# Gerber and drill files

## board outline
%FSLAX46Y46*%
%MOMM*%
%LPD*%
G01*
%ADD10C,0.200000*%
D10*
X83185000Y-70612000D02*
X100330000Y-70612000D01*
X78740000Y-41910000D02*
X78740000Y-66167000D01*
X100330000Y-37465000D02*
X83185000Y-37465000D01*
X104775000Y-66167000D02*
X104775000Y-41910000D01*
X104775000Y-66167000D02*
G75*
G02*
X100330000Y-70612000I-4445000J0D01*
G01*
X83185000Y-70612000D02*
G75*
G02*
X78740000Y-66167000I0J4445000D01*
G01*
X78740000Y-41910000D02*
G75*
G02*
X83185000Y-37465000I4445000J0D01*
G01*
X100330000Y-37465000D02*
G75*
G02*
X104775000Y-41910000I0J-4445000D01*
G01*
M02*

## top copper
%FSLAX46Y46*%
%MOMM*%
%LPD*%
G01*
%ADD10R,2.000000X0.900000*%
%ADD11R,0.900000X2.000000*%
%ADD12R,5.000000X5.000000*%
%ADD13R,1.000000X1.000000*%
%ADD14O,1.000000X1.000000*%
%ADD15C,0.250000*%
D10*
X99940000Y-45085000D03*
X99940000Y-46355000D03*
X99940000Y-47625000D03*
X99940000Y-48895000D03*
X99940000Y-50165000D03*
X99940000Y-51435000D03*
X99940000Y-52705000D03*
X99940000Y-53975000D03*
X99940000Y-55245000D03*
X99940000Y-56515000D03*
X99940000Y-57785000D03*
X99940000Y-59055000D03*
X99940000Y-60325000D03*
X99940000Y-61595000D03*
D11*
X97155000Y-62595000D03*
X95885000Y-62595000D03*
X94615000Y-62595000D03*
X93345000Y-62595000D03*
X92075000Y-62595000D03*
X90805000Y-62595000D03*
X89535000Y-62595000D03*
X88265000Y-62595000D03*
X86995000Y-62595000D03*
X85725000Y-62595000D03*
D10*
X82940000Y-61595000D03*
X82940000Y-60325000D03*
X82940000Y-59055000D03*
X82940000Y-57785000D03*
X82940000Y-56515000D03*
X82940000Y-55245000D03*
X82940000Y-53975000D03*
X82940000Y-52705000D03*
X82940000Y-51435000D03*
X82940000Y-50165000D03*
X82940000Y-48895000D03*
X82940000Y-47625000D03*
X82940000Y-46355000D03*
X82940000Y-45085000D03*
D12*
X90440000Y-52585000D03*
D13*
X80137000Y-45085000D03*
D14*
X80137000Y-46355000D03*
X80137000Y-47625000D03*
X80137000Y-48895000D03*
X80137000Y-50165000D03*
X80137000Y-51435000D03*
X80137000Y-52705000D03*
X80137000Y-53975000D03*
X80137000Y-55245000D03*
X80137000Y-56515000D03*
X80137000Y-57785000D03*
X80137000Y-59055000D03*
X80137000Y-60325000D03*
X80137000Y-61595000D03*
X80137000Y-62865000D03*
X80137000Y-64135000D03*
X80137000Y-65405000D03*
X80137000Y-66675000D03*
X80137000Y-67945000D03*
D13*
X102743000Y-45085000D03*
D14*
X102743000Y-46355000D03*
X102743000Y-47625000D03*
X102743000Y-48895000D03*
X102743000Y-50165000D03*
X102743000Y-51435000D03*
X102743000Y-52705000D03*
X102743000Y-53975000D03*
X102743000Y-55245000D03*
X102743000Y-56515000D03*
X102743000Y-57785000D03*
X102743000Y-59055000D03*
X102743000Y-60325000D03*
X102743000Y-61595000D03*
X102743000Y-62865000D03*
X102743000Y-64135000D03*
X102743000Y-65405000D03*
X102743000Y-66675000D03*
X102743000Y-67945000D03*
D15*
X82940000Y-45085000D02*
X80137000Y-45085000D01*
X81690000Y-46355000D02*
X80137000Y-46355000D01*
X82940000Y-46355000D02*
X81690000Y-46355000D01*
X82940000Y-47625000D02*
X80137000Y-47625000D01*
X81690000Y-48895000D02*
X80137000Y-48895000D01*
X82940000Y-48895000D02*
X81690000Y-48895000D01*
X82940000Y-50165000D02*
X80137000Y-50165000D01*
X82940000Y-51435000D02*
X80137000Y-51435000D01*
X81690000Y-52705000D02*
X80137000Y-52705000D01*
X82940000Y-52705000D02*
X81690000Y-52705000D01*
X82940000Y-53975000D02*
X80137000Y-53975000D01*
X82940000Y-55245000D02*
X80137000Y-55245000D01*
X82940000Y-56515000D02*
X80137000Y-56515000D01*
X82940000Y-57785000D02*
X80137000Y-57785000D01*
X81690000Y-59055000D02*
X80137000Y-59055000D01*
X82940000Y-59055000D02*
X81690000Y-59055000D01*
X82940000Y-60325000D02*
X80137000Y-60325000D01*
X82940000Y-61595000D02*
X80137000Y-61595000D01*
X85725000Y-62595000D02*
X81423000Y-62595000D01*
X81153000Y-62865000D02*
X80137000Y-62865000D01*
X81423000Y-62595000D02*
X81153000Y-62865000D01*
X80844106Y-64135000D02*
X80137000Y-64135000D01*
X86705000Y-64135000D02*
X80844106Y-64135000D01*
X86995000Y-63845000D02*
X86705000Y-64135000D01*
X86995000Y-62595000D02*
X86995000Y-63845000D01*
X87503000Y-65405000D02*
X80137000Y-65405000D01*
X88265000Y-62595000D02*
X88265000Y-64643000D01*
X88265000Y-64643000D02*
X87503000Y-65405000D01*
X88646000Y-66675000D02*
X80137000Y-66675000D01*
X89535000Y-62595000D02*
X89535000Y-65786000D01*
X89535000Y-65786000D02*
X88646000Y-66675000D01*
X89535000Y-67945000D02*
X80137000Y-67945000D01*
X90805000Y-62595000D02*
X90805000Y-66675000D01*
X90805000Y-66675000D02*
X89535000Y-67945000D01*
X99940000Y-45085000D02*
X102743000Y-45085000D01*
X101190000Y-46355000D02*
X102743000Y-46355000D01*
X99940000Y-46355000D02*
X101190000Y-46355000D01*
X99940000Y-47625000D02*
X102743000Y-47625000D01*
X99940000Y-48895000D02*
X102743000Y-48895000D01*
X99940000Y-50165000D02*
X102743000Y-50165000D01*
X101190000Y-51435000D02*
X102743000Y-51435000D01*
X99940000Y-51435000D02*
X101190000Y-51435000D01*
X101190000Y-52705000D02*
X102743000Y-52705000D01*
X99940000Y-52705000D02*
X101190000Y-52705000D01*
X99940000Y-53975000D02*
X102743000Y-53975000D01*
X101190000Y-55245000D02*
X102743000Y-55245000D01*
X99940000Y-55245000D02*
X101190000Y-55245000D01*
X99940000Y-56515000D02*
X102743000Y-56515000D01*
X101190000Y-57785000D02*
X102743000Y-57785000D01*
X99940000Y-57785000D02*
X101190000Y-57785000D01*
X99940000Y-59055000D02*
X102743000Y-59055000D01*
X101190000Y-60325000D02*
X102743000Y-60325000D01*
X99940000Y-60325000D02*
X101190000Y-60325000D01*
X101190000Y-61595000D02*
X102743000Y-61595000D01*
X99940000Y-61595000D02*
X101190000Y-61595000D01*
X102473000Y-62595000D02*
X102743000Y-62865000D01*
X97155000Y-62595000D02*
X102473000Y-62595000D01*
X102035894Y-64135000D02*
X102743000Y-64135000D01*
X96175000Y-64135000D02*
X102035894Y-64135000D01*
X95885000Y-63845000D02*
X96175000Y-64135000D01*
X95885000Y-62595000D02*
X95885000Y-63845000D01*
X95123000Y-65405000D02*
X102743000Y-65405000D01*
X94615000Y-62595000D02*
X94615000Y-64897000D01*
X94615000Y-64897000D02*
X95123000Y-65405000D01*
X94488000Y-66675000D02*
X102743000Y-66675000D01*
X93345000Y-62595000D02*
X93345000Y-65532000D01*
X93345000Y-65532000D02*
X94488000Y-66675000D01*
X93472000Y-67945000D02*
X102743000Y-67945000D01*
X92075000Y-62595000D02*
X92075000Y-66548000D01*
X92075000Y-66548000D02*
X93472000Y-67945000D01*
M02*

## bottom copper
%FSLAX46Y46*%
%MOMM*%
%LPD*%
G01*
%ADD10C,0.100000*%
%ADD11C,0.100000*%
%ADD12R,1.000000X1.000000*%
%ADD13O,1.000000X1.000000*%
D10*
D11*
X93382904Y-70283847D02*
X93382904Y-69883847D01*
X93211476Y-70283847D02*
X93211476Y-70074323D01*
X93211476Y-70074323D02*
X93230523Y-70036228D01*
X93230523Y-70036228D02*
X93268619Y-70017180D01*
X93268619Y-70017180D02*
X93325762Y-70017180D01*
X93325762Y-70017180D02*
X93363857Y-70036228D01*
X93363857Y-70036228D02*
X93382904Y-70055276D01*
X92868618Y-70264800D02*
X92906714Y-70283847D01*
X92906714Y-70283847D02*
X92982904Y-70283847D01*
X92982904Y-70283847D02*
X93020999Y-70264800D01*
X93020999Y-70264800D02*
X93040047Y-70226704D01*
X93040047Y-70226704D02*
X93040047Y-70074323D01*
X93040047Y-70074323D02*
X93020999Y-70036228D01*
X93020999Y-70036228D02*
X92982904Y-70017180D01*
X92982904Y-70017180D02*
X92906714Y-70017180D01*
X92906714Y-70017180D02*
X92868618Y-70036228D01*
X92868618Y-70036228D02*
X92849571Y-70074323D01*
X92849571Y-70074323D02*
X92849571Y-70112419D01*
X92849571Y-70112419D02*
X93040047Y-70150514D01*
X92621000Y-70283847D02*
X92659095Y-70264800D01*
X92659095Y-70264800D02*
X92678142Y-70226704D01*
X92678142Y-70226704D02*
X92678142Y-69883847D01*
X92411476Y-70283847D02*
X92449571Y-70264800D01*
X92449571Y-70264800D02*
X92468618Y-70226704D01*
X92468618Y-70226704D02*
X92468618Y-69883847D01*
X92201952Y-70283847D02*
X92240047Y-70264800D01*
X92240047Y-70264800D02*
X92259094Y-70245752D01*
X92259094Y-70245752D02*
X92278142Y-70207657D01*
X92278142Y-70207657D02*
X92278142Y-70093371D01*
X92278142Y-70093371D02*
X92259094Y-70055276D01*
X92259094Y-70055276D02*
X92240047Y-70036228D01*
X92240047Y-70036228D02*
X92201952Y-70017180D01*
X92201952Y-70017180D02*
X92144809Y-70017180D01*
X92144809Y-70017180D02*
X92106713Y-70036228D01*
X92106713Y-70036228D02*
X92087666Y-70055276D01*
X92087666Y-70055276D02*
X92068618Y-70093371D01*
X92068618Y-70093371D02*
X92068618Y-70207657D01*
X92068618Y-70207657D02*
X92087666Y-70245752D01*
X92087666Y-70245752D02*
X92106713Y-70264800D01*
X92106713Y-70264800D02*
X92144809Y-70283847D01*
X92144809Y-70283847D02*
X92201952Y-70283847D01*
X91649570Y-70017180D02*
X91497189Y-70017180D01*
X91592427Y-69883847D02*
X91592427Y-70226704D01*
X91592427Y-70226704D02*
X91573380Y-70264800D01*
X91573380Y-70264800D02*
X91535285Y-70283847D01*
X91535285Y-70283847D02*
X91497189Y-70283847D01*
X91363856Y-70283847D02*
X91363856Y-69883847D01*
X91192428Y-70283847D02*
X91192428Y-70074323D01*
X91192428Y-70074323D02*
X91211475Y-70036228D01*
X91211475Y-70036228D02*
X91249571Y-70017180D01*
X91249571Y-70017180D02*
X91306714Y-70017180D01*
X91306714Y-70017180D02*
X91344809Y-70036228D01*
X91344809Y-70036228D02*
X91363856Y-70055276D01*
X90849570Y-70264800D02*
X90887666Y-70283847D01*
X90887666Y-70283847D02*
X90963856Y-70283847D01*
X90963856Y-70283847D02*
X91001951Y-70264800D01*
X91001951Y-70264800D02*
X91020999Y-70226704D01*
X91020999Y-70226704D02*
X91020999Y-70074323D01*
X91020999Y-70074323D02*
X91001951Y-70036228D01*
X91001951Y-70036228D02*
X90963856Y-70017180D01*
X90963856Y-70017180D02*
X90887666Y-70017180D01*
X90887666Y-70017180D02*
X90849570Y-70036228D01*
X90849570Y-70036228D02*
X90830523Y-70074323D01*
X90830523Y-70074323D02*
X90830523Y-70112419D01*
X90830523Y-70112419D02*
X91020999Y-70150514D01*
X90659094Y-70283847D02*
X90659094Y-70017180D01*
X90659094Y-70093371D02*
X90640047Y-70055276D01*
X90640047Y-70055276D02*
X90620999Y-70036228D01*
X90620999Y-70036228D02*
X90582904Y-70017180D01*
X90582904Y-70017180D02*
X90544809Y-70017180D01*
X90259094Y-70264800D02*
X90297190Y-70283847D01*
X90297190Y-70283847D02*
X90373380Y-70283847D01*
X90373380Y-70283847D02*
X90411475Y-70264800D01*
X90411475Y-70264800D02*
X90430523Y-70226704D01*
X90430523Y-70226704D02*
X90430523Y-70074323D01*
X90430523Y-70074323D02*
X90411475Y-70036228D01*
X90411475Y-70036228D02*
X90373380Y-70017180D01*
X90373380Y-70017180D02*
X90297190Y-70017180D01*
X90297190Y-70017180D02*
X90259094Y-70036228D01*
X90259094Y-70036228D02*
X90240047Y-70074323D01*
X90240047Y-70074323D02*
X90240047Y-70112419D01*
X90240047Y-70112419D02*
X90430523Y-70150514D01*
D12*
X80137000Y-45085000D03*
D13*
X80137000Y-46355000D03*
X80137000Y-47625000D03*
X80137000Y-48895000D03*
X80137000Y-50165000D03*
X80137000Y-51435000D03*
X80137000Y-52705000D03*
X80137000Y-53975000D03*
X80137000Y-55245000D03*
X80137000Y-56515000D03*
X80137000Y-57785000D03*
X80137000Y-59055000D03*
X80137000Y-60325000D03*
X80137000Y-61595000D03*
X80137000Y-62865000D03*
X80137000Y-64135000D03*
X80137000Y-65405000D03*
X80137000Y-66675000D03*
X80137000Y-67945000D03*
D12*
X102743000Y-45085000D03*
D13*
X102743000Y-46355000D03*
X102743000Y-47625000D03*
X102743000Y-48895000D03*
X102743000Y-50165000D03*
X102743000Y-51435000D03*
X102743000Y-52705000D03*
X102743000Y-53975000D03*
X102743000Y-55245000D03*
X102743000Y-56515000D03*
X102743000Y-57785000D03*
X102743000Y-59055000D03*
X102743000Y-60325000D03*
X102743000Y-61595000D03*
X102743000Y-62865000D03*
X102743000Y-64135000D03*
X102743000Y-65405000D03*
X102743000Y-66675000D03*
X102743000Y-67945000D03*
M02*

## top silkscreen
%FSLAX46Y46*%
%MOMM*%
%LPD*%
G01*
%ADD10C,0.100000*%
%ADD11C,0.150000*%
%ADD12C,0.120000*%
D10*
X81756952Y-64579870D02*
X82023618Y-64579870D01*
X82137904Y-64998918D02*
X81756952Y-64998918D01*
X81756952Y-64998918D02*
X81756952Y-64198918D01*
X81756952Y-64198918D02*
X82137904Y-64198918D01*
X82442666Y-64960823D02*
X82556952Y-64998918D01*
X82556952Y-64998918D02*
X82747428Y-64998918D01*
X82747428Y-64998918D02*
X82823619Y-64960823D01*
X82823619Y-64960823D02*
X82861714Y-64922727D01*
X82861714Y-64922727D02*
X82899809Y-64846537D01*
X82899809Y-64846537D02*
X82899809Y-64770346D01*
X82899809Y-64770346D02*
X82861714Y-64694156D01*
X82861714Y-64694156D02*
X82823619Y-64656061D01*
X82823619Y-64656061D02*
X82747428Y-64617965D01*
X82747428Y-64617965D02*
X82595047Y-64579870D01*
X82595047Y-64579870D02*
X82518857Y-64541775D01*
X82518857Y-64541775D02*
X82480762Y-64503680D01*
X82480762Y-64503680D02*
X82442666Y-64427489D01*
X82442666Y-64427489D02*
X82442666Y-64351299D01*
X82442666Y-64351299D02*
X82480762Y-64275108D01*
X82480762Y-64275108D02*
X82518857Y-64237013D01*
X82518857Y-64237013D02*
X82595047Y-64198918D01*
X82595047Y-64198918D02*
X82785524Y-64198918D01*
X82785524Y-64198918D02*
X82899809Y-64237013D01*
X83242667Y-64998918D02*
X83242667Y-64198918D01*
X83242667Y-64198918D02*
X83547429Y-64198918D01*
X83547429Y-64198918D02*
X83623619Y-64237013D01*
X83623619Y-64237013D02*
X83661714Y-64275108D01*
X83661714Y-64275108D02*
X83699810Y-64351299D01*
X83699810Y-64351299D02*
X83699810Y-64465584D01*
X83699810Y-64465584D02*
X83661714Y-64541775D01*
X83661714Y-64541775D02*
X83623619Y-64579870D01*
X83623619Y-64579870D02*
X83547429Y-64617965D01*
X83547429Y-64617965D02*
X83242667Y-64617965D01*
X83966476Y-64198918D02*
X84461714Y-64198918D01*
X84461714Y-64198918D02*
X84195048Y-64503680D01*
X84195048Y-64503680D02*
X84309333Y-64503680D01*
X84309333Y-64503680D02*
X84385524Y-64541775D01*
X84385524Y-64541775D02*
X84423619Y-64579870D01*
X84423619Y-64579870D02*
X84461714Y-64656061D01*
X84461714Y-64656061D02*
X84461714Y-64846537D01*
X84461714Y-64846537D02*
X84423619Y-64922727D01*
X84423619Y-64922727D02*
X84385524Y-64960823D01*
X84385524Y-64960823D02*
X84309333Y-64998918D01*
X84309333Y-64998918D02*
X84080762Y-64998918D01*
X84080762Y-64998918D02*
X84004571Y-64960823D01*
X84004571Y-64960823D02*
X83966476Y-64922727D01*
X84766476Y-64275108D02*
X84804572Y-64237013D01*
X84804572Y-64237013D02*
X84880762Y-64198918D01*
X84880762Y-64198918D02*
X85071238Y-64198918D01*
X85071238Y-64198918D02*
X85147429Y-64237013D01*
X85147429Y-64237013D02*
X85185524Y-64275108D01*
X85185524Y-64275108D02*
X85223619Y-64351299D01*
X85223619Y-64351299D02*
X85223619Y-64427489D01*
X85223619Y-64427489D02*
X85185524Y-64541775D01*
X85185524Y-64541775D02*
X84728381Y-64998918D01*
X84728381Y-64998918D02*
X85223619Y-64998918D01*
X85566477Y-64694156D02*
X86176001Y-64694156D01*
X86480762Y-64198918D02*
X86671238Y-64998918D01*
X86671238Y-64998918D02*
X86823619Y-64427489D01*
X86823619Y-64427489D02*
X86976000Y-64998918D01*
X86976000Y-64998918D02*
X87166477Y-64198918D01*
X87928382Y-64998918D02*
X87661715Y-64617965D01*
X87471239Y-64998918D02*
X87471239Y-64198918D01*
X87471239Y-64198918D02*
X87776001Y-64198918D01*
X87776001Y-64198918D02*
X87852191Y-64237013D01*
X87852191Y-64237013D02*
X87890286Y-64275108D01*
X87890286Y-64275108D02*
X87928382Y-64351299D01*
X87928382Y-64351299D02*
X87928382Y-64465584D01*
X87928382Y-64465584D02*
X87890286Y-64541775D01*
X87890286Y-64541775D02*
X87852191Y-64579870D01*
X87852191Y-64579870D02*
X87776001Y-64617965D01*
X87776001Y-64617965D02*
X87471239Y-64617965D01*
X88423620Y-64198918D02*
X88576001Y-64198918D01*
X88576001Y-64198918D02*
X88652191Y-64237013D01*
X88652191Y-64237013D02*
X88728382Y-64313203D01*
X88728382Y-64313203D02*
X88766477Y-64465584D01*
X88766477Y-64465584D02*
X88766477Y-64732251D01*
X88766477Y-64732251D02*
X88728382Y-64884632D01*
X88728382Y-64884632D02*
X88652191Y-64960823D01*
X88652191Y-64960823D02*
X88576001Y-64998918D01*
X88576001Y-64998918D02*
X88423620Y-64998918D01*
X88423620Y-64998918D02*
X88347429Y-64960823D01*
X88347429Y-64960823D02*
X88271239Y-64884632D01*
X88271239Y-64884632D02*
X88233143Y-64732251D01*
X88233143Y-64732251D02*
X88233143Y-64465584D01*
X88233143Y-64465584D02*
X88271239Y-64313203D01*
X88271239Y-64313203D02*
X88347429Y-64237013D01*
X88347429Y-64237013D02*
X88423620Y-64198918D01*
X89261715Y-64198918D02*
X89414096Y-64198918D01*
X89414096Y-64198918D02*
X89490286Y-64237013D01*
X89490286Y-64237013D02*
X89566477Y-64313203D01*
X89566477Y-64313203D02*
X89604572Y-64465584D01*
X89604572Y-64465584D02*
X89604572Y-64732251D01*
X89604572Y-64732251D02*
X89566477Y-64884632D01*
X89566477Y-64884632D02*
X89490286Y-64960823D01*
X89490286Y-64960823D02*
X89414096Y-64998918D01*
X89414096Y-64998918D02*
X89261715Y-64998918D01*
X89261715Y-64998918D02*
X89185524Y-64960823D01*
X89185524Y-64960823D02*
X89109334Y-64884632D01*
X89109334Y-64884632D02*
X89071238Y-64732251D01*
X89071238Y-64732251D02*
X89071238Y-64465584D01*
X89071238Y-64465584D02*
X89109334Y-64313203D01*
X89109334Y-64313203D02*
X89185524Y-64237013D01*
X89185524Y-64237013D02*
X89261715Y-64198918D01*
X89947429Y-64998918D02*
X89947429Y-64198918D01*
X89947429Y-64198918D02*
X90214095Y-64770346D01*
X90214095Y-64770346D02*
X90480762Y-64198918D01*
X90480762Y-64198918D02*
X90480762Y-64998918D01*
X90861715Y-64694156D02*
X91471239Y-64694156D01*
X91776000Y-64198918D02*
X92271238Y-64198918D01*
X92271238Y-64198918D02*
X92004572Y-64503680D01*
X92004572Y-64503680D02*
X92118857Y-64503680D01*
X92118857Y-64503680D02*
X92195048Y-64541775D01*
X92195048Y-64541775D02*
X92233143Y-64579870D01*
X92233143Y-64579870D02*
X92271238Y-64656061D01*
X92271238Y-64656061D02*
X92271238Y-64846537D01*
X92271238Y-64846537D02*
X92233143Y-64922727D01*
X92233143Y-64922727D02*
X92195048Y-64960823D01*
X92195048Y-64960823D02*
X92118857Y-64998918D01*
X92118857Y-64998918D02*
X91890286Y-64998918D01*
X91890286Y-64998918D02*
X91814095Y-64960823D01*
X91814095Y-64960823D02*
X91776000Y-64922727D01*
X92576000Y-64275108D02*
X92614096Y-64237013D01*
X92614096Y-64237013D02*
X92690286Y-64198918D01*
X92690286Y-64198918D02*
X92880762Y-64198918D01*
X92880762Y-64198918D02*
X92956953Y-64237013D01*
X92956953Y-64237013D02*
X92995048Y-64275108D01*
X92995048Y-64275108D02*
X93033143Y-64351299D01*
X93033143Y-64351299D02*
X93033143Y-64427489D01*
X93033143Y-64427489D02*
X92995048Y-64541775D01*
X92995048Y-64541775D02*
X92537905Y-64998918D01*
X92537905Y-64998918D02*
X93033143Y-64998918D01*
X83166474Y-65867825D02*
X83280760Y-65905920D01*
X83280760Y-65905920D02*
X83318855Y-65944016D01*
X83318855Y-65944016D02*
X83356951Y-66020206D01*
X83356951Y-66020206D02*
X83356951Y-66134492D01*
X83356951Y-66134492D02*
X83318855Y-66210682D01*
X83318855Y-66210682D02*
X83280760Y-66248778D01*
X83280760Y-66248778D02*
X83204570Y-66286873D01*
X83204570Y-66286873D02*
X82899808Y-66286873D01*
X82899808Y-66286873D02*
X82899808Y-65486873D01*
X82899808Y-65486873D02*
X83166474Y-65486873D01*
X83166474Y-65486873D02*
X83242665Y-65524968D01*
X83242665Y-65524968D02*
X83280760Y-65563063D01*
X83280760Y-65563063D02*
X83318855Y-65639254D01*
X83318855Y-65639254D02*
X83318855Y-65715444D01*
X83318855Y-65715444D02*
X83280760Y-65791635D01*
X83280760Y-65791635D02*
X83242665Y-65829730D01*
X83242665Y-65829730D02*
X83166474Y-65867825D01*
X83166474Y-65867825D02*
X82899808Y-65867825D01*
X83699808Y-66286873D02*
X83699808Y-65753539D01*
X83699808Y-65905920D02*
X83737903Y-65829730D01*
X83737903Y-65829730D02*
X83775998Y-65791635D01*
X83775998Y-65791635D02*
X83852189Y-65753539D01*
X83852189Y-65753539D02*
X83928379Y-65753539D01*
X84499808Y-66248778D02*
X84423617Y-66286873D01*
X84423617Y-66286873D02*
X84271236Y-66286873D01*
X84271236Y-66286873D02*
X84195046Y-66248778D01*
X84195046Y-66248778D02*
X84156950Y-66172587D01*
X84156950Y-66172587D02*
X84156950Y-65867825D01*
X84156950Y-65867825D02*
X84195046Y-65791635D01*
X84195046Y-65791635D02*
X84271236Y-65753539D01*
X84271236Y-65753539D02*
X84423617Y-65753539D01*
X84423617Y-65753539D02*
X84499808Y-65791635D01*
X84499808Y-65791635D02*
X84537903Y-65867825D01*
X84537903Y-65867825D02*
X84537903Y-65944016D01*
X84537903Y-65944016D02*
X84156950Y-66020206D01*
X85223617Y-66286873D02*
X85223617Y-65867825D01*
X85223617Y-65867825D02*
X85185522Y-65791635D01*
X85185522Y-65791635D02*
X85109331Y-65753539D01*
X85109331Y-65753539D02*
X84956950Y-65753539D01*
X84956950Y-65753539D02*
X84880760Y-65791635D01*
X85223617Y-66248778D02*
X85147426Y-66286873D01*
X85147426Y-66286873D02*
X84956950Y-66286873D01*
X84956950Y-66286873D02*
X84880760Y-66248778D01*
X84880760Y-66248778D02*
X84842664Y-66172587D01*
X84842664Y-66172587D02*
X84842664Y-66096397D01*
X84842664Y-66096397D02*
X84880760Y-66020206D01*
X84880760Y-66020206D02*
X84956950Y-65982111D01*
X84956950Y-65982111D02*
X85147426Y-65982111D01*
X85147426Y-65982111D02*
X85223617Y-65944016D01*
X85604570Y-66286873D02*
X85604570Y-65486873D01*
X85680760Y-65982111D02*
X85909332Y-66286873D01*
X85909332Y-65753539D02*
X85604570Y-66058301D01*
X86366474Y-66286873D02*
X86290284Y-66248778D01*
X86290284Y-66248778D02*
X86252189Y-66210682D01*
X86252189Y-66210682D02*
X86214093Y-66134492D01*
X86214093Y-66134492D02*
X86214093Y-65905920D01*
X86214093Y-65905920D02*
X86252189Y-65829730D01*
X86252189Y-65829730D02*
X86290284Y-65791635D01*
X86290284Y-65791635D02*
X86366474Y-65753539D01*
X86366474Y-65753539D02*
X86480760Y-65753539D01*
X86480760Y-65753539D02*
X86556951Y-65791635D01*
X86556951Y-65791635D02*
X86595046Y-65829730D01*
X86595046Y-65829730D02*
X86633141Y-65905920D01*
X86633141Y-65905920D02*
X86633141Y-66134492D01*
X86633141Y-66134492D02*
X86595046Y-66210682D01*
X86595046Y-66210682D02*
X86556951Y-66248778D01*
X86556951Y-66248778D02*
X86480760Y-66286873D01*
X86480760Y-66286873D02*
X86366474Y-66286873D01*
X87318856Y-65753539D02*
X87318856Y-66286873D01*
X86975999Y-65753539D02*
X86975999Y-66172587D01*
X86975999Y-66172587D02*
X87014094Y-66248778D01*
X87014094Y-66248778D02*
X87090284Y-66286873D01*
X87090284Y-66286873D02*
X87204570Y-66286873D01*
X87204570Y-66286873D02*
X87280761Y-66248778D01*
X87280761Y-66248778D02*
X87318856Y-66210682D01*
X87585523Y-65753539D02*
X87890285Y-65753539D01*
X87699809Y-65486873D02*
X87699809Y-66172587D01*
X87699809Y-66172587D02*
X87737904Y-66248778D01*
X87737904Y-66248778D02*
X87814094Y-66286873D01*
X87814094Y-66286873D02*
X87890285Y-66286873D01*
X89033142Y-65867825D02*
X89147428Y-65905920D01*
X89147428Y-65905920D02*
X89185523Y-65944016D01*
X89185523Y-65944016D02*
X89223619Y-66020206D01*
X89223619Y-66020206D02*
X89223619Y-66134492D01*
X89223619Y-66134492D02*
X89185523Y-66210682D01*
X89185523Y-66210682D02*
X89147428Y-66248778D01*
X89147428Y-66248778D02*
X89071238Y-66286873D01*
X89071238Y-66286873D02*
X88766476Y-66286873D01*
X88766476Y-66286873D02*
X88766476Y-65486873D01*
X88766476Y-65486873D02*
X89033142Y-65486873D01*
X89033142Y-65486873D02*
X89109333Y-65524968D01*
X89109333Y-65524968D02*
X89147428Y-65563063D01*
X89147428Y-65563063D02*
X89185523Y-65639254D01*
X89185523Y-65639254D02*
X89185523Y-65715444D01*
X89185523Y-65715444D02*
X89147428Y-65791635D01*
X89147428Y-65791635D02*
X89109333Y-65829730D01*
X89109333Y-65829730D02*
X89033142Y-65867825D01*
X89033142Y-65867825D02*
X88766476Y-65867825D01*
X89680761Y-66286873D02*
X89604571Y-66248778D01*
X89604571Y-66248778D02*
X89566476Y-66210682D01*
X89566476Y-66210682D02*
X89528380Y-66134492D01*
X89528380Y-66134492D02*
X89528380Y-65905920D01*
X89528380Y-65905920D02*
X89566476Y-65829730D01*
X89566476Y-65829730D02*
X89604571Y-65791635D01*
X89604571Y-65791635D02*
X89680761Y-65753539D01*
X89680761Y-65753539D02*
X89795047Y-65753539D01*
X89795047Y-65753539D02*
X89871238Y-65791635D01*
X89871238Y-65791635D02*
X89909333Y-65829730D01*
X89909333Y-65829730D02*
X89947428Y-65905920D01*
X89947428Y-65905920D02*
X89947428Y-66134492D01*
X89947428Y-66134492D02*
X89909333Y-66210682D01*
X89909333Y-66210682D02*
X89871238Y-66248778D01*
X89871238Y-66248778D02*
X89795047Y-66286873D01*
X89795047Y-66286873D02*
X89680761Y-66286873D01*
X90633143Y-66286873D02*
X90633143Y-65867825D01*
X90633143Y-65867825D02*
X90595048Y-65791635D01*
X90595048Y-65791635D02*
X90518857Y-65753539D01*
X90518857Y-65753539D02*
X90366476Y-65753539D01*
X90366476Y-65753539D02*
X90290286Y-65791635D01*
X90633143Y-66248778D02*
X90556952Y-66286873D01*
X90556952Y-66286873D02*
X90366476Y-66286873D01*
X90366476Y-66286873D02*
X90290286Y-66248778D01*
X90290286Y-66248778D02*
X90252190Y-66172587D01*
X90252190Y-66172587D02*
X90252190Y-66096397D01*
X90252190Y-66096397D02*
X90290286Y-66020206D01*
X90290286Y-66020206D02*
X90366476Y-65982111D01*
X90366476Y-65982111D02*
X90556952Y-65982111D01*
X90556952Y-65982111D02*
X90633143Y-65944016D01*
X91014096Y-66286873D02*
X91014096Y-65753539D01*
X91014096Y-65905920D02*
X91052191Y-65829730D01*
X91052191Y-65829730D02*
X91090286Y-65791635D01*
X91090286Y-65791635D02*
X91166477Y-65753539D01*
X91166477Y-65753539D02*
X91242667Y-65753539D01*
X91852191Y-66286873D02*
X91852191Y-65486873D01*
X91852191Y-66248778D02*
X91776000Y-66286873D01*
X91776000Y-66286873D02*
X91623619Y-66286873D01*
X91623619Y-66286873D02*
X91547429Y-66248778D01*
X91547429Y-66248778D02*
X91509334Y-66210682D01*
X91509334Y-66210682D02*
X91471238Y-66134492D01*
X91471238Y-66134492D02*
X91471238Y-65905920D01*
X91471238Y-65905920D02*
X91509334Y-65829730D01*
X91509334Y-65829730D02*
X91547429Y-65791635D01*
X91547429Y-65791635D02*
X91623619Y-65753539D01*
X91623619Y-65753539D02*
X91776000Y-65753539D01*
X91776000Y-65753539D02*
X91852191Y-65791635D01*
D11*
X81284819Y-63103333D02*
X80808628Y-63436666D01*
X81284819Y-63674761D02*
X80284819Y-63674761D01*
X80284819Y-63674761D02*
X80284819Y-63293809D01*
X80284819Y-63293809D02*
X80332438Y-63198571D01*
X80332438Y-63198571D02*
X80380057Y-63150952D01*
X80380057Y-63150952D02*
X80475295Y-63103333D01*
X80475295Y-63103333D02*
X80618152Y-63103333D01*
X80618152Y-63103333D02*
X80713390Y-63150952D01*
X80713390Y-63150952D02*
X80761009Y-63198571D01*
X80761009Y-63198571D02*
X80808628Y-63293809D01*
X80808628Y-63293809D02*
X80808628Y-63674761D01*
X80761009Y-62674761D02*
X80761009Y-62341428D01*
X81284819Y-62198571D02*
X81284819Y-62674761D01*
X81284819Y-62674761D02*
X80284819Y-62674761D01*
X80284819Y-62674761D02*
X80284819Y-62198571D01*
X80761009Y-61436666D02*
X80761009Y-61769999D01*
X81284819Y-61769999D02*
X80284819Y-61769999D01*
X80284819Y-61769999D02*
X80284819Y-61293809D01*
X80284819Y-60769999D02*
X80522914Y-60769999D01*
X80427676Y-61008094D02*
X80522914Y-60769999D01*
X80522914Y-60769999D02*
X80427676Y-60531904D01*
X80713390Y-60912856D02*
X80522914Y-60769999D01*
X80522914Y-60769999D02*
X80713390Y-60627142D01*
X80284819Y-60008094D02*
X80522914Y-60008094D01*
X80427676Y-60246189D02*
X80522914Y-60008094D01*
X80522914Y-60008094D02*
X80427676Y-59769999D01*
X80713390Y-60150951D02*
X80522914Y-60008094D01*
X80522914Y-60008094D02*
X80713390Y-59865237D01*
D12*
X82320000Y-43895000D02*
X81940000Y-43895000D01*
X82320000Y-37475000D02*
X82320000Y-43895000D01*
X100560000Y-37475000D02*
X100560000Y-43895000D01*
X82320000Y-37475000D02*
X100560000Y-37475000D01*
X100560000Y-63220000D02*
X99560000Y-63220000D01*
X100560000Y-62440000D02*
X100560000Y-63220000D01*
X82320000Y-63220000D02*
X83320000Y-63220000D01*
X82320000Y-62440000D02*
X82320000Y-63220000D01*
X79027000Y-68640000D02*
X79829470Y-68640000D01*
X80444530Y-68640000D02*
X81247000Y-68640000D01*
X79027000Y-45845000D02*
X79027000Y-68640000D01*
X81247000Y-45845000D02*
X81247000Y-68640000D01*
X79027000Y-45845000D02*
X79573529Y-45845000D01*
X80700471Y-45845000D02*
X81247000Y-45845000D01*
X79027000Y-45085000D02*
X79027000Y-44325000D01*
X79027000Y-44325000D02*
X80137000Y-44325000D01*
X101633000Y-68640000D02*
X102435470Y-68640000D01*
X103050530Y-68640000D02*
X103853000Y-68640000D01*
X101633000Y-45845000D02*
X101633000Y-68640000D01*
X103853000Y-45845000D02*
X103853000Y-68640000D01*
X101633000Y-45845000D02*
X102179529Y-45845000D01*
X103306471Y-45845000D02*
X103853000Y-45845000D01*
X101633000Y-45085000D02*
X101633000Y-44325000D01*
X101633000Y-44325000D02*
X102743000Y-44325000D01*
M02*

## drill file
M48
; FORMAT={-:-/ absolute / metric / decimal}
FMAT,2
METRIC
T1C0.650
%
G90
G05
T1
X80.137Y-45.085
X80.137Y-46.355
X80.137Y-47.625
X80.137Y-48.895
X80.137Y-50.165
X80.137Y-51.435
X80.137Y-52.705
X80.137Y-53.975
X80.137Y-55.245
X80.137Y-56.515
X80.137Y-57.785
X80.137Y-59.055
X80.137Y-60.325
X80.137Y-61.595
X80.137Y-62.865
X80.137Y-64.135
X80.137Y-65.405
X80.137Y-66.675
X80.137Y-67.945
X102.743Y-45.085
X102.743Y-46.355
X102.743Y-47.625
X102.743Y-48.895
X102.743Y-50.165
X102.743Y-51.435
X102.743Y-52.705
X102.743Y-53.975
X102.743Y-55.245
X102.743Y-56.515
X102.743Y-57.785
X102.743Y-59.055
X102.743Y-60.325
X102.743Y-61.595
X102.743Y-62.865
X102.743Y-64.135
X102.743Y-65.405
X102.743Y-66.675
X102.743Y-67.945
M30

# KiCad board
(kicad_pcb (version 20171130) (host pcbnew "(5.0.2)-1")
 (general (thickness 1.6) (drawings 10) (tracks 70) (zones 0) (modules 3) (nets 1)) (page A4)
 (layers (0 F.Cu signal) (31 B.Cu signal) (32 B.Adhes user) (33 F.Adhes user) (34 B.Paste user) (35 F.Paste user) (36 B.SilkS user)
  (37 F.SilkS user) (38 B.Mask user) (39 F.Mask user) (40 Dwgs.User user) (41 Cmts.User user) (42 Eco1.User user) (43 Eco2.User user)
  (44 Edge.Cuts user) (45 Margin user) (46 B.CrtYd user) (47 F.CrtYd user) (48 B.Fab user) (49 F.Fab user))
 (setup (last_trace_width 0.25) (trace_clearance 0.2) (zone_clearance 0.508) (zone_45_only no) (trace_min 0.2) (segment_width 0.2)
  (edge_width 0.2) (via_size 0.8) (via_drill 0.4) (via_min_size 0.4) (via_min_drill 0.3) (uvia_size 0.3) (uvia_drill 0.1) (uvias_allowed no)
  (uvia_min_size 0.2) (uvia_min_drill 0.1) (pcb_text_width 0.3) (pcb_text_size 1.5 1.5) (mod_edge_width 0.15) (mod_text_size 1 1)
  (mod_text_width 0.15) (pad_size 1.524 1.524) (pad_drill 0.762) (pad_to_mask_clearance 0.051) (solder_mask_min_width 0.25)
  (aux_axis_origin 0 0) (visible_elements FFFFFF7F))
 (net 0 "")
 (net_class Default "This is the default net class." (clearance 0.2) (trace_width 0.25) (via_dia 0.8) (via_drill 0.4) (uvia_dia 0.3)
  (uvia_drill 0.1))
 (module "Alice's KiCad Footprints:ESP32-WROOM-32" (layer F.Cu) (at 91.44 53.34)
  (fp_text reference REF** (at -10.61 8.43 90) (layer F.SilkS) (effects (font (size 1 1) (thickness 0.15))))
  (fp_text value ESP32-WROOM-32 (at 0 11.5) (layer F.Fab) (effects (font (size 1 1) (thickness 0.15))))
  (fp_line (start -9.12 -9.445) (end -9.5 -9.445) (layer F.SilkS) (width 0.12))
  (fp_line (start -9.12 -15.865) (end -9.12 -9.445) (layer F.SilkS) (width 0.12))
  (fp_line (start 9.12 -15.865) (end 9.12 -9.445) (layer F.SilkS) (width 0.12))
  (fp_line (start -9.12 -15.865) (end 9.12 -15.865) (layer F.SilkS) (width 0.12))
  (fp_line (start 9.12 9.88) (end 8.12 9.88) (layer F.SilkS) (width 0.12))
  (fp_line (start 9.12 9.1) (end 9.12 9.88) (layer F.SilkS) (width 0.12))
  (fp_line (start -9.12 9.88) (end -8.12 9.88) (layer F.SilkS) (width 0.12))
  (fp_line (start -9.12 9.1) (end -9.12 9.88) (layer F.SilkS) (width 0.12))
  (pad 38 smd rect (at 8.5 -8.255) (size 2 0.9) (layers F.Cu F.Paste F.Mask))
  (pad 37 smd rect (at 8.5 -6.985) (size 2 0.9) (layers F.Cu F.Paste F.Mask))
  (pad 36 smd rect (at 8.5 -5.715) (size 2 0.9) (layers F.Cu F.Paste F.Mask))
  (pad 35 smd rect (at 8.5 -4.445) (size 2 0.9) (layers F.Cu F.Paste F.Mask))
  (pad 34 smd rect (at 8.5 -3.175) (size 2 0.9) (layers F.Cu F.Paste F.Mask))
  (pad 33 smd rect (at 8.5 -1.905) (size 2 0.9) (layers F.Cu F.Paste F.Mask))
  (pad 32 smd rect (at 8.5 -0.635) (size 2 0.9) (layers F.Cu F.Paste F.Mask))
  (pad 31 smd rect (at 8.5 0.635) (size 2 0.9) (layers F.Cu F.Paste F.Mask))
  (pad 30 smd rect (at 8.5 1.905) (size 2 0.9) (layers F.Cu F.Paste F.Mask))
  (pad 29 smd rect (at 8.5 3.175) (size 2 0.9) (layers F.Cu F.Paste F.Mask))
  (pad 28 smd rect (at 8.5 4.445) (size 2 0.9) (layers F.Cu F.Paste F.Mask))
  (pad 27 smd rect (at 8.5 5.715) (size 2 0.9) (layers F.Cu F.Paste F.Mask))
  (pad 26 smd rect (at 8.5 6.985) (size 2 0.9) (layers F.Cu F.Paste F.Mask))
  (pad 25 smd rect (at 8.5 8.255) (size 2 0.9) (layers F.Cu F.Paste F.Mask))
  (pad 24 smd rect (at 5.715 9.255 90) (size 2 0.9) (layers F.Cu F.Paste F.Mask))
  (pad 23 smd rect (at 4.445 9.255 90) (size 2 0.9) (layers F.Cu F.Paste F.Mask))
  (pad 22 smd rect (at 3.175 9.255 90) (size 2 0.9) (layers F.Cu F.Paste F.Mask))
  (pad 21 smd rect (at 1.905 9.255 90) (size 2 0.9) (layers F.Cu F.Paste F.Mask))
  (pad 20 smd rect (at 0.635 9.255 90) (size 2 0.9) (layers F.Cu F.Paste F.Mask))
  (pad 19 smd rect (at -0.635 9.255 90) (size 2 0.9) (layers F.Cu F.Paste F.Mask))
  (pad 18 smd rect (at -1.905 9.255 90) (size 2 0.9) (layers F.Cu F.Paste F.Mask))
  (pad 17 smd rect (at -3.175 9.255 90) (size 2 0.9) (layers F.Cu F.Paste F.Mask))
  (pad 16 smd rect (at -4.445 9.255 90) (size 2 0.9) (layers F.Cu F.Paste F.Mask))
  (pad 15 smd rect (at -5.715 9.255 90) (size 2 0.9) (layers F.Cu F.Paste F.Mask))
  (pad 14 smd rect (at -8.5 8.255) (size 2 0.9) (layers F.Cu F.Paste F.Mask))
  (pad 13 smd rect (at -8.5 6.985) (size 2 0.9) (layers F.Cu F.Paste F.Mask))
  (pad 12 smd rect (at -8.5 5.715) (size 2 0.9) (layers F.Cu F.Paste F.Mask))
  (pad 11 smd rect (at -8.5 4.445) (size 2 0.9) (layers F.Cu F.Paste F.Mask))
  (pad 10 smd rect (at -8.5 3.175) (size 2 0.9) (layers F.Cu F.Paste F.Mask))
  (pad 9 smd rect (at -8.5 1.905) (size 2 0.9) (layers F.Cu F.Paste F.Mask))
  (pad 8 smd rect (at -8.5 0.635) (size 2 0.9) (layers F.Cu F.Paste F.Mask))
  (pad 7 smd rect (at -8.5 -0.635) (size 2 0.9) (layers F.Cu F.Paste F.Mask))
  (pad 6 smd rect (at -8.5 -1.905) (size 2 0.9) (layers F.Cu F.Paste F.Mask))
  (pad 5 smd rect (at -8.5 -3.175) (size 2 0.9) (layers F.Cu F.Paste F.Mask))
  (pad 4 smd rect (at -8.5 -4.445) (size 2 0.9) (layers F.Cu F.Paste F.Mask))
  (pad 3 smd rect (at -8.5 -5.715) (size 2 0.9) (layers F.Cu F.Paste F.Mask))
  (pad 2 smd rect (at -8.5 -6.985) (size 2 0.9) (layers F.Cu F.Paste F.Mask))
  (pad 1 smd rect (at -8.5 -8.255) (size 2 0.9) (layers F.Cu F.Paste F.Mask))
  (pad 39 smd rect (at -1 -0.755) (size 5 5) (layers F.Cu F.Paste F.Mask)))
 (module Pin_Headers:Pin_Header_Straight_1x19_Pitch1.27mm (layer F.Cu) (at 80.137 45.085)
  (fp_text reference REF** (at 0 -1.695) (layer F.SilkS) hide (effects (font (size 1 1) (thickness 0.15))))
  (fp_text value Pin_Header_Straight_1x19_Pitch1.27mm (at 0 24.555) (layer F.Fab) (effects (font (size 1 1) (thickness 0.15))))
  (fp_line (start -1.11 23.555) (end -0.30753 23.555) (layer F.SilkS) (width 0.12))
  (fp_line (start 0.30753 23.555) (end 1.11 23.555) (layer F.SilkS) (width 0.12))
  (fp_line (start -1.11 0.76) (end -1.11 23.555) (layer F.SilkS) (width 0.12))
  (fp_line (start 1.11 0.76) (end 1.11 23.555) (layer F.SilkS) (width 0.12))
  (fp_line (start -1.11 0.76) (end -0.563471 0.76) (layer F.SilkS) (width 0.12))
  (fp_line (start 0.563471 0.76) (end 1.11 0.76) (layer F.SilkS) (width 0.12))
  (fp_line (start -1.11 0) (end -1.11 -0.76) (layer F.SilkS) (width 0.12))
  (fp_line (start -1.11 -0.76) (end 0 -0.76) (layer F.SilkS) (width 0.12))
  (pad 1 thru_hole rect (at 0 0) (size 1 1) (drill 0.65) (layers *.Cu *.Mask))
  (pad 2 thru_hole oval (at 0 1.27) (size 1 1) (drill 0.65) (layers *.Cu *.Mask))
  (pad 3 thru_hole oval (at 0 2.54) (size 1 1) (drill 0.65) (layers *.Cu *.Mask))
  (pad 4 thru_hole oval (at 0 3.81) (size 1 1) (drill 0.65) (layers *.Cu *.Mask))
  (pad 5 thru_hole oval (at 0 5.08) (size 1 1) (drill 0.65) (layers *.Cu *.Mask))
  (pad 6 thru_hole oval (at 0 6.35) (size 1 1) (drill 0.65) (layers *.Cu *.Mask))
  (pad 7 thru_hole oval (at 0 7.62) (size 1 1) (drill 0.65) (layers *.Cu *.Mask))
  (pad 8 thru_hole oval (at 0 8.89) (size 1 1) (drill 0.65) (layers *.Cu *.Mask))
  (pad 9 thru_hole oval (at 0 10.16) (size 1 1) (drill 0.65) (layers *.Cu *.Mask))
  (pad 10 thru_hole oval (at 0 11.43) (size 1 1) (drill 0.65) (layers *.Cu *.Mask))
  (pad 11 thru_hole oval (at 0 12.7) (size 1 1) (drill 0.65) (layers *.Cu *.Mask))
  (pad 12 thru_hole oval (at 0 13.97) (size 1 1) (drill 0.65) (layers *.Cu *.Mask))
  (pad 13 thru_hole oval (at 0 15.24) (size 1 1) (drill 0.65) (layers *.Cu *.Mask))
  (pad 14 thru_hole oval (at 0 16.51) (size 1 1) (drill 0.65) (layers *.Cu *.Mask))
  (pad 15 thru_hole oval (at 0 17.78) (size 1 1) (drill 0.65) (layers *.Cu *.Mask))
  (pad 16 thru_hole oval (at 0 19.05) (size 1 1) (drill 0.65) (layers *.Cu *.Mask))
  (pad 17 thru_hole oval (at 0 20.32) (size 1 1) (drill 0.65) (layers *.Cu *.Mask))
  (pad 18 thru_hole oval (at 0 21.59) (size 1 1) (drill 0.65) (layers *.Cu *.Mask))
  (pad 19 thru_hole oval (at 0 22.86) (size 1 1) (drill 0.65) (layers *.Cu *.Mask)))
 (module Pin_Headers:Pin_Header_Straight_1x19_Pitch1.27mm (layer F.Cu) (at 102.743 45.085)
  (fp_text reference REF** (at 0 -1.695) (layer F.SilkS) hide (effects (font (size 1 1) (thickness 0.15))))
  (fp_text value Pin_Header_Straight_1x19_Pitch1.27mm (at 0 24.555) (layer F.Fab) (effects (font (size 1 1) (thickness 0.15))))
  (fp_line (start -1.11 23.555) (end -0.30753 23.555) (layer F.SilkS) (width 0.12))
  (fp_line (start 0.30753 23.555) (end 1.11 23.555) (layer F.SilkS) (width 0.12))
  (fp_line (start -1.11 0.76) (end -1.11 23.555) (layer F.SilkS) (width 0.12))
  (fp_line (start 1.11 0.76) (end 1.11 23.555) (layer F.SilkS) (width 0.12))
  (fp_line (start -1.11 0.76) (end -0.563471 0.76) (layer F.SilkS) (width 0.12))
  (fp_line (start 0.563471 0.76) (end 1.11 0.76) (layer F.SilkS) (width 0.12))
  (fp_line (start -1.11 0) (end -1.11 -0.76) (layer F.SilkS) (width 0.12))
  (fp_line (start -1.11 -0.76) (end 0 -0.76) (layer F.SilkS) (width 0.12))
  (pad 1 thru_hole rect (at 0 0) (size 1 1) (drill 0.65) (layers *.Cu *.Mask))
  (pad 2 thru_hole oval (at 0 1.27) (size 1 1) (drill 0.65) (layers *.Cu *.Mask))
  (pad 3 thru_hole oval (at 0 2.54) (size 1 1) (drill 0.65) (layers *.Cu *.Mask))
  (pad 4 thru_hole oval (at 0 3.81) (size 1 1) (drill 0.65) (layers *.Cu *.Mask))
  (pad 5 thru_hole oval (at 0 5.08) (size 1 1) (drill 0.65) (layers *.Cu *.Mask))
  (pad 6 thru_hole oval (at 0 6.35) (size 1 1) (drill 0.65) (layers *.Cu *.Mask))
  (pad 7 thru_hole oval (at 0 7.62) (size 1 1) (drill 0.65) (layers *.Cu *.Mask))
  (pad 8 thru_hole oval (at 0 8.89) (size 1 1) (drill 0.65) (layers *.Cu *.Mask))
  (pad 9 thru_hole oval (at 0 10.16) (size 1 1) (drill 0.65) (layers *.Cu *.Mask))
  (pad 10 thru_hole oval (at 0 11.43) (size 1 1) (drill 0.65) (layers *.Cu *.Mask))
  (pad 11 thru_hole oval (at 0 12.7) (size 1 1) (drill 0.65) (layers *.Cu *.Mask))
  (pad 12 thru_hole oval (at 0 13.97) (size 1 1) (drill 0.65) (layers *.Cu *.Mask))
  (pad 13 thru_hole oval (at 0 15.24) (size 1 1) (drill 0.65) (layers *.Cu *.Mask))
  (pad 14 thru_hole oval (at 0 16.51) (size 1 1) (drill 0.65) (layers *.Cu *.Mask))
  (pad 15 thru_hole oval (at 0 17.78) (size 1 1) (drill 0.65) (layers *.Cu *.Mask))
  (pad 16 thru_hole oval (at 0 19.05) (size 1 1) (drill 0.65) (layers *.Cu *.Mask))
  (pad 17 thru_hole oval (at 0 20.32) (size 1 1) (drill 0.65) (layers *.Cu *.Mask))
  (pad 18 thru_hole oval (at 0 21.59) (size 1 1) (drill 0.65) (layers *.Cu *.Mask))
  (pad 19 thru_hole oval (at 0 22.86) (size 1 1) (drill 0.65) (layers *.Cu *.Mask)))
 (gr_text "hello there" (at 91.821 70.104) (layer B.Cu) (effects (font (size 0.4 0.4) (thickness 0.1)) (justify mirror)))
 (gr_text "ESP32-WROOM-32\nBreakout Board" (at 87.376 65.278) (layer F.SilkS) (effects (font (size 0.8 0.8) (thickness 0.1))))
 (gr_line (start 83.185 70.612) (end 100.33 70.612) (layer Edge.Cuts) (width 0.2))
 (gr_line (start 78.74 41.91) (end 78.74 66.167) (layer Edge.Cuts) (width 0.2))
 (gr_line (start 100.33 37.465) (end 83.185 37.465) (layer Edge.Cuts) (width 0.2))
 (gr_line (start 104.775 66.167) (end 104.775 41.91) (layer Edge.Cuts) (width 0.2))
 (gr_arc (start 100.33 66.167) (end 100.33 70.612) (angle -90) (layer Edge.Cuts) (width 0.2))
 (gr_arc (start 83.185 66.167) (end 78.74 66.167) (angle -90) (layer Edge.Cuts) (width 0.2))
 (gr_arc (start 83.185 41.91) (end 83.185 37.465) (angle -90) (layer Edge.Cuts) (width 0.2))
 (gr_arc (start 100.33 41.91) (end 104.775 41.91) (angle -90) (layer Edge.Cuts) (width 0.2))
 (segment (start 82.94 45.085) (end 80.137 45.085) (width 0.25) (layer F.Cu) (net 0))
 (segment (start 81.69 46.355) (end 80.137 46.355) (width 0.25) (layer F.Cu) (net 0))
 (segment (start 82.94 46.355) (end 81.69 46.355) (width 0.25) (layer F.Cu) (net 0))
 (segment (start 82.94 47.625) (end 80.137 47.625) (width 0.25) (layer F.Cu) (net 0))
 (segment (start 81.69 48.895) (end 80.137 48.895) (width 0.25) (layer F.Cu) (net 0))
 (segment (start 82.94 48.895) (end 81.69 48.895) (width 0.25) (layer F.Cu) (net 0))
 (segment (start 82.94 50.165) (end 80.137 50.165) (width 0.25) (layer F.Cu) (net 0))
 (segment (start 82.94 51.435) (end 80.137 51.435) (width 0.25) (layer F.Cu) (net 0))
 (segment (start 81.69 52.705) (end 80.137 52.705) (width 0.25) (layer F.Cu) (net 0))
 (segment (start 82.94 52.705) (end 81.69 52.705) (width 0.25) (layer F.Cu) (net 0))
 (segment (start 82.94 53.975) (end 80.137 53.975) (width 0.25) (layer F.Cu) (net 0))
 (segment (start 82.94 55.245) (end 80.137 55.245) (width 0.25) (layer F.Cu) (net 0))
 (segment (start 82.94 56.515) (end 80.137 56.515) (width 0.25) (layer F.Cu) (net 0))
 (segment (start 82.94 57.785) (end 80.137 57.785) (width 0.25) (layer F.Cu) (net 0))
 (segment (start 81.69 59.055) (end 80.137 59.055) (width 0.25) (layer F.Cu) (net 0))
 (segment (start 82.94 59.055) (end 81.69 59.055) (width 0.25) (layer F.Cu) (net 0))
 (segment (start 82.94 60.325) (end 80.137 60.325) (width 0.25) (layer F.Cu) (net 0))
 (segment (start 82.94 61.595) (end 80.137 61.595) (width 0.25) (layer F.Cu) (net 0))
 (segment (start 85.725 62.595) (end 81.423 62.595) (width 0.25) (layer F.Cu) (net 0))
 (segment (start 81.153 62.865) (end 80.137 62.865) (width 0.25) (layer F.Cu) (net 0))
 (segment (start 81.423 62.595) (end 81.153 62.865) (width 0.25) (layer F.Cu) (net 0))
 (segment (start 80.844106 64.135) (end 80.137 64.135) (width 0.25) (layer F.Cu) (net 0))
 (segment (start 86.705 64.135) (end 80.844106 64.135) (width 0.25) (layer F.Cu) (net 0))
 (segment (start 86.995 63.845) (end 86.705 64.135) (width 0.25) (layer F.Cu) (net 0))
 (segment (start 86.995 62.595) (end 86.995 63.845) (width 0.25) (layer F.Cu) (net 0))
 (segment (start 87.503 65.405) (end 80.137 65.405) (width 0.25) (layer F.Cu) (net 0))
 (segment (start 88.265 62.595) (end 88.265 64.643) (width 0.25) (layer F.Cu) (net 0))
 (segment (start 88.265 64.643) (end 87.503 65.405) (width 0.25) (layer F.Cu) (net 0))
 (segment (start 88.646 66.675) (end 80.137 66.675) (width 0.25) (layer F.Cu) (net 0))
 (segment (start 89.535 62.595) (end 89.535 65.786) (width 0.25) (layer F.Cu) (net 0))
 (segment (start 89.535 65.786) (end 88.646 66.675) (width 0.25) (layer F.Cu) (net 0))
 (segment (start 89.535 67.945) (end 80.137 67.945) (width 0.25) (layer F.Cu) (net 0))
 (segment (start 90.805 62.595) (end 90.805 66.675) (width 0.25) (layer F.Cu) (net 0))
 (segment (start 90.805 66.675) (end 89.535 67.945) (width 0.25) (layer F.Cu) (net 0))
 (segment (start 99.94 45.085) (end 102.743 45.085) (width 0.25) (layer F.Cu) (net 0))
 (segment (start 101.19 46.355) (end 102.743 46.355) (width 0.25) (layer F.Cu) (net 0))
 (segment (start 99.94 46.355) (end 101.19 46.355) (width 0.25) (layer F.Cu) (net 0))
 (segment (start 99.94 47.625) (end 102.743 47.625) (width 0.25) (layer F.Cu) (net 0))
 (segment (start 99.94 48.895) (end 102.743 48.895) (width 0.25) (layer F.Cu) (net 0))
 (segment (start 99.94 50.165) (end 102.743 50.165) (width 0.25) (layer F.Cu) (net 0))
 (segment (start 101.19 51.435) (end 102.743 51.435) (width 0.25) (layer F.Cu) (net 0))
 (segment (start 99.94 51.435) (end 101.19 51.435) (width 0.25) (layer F.Cu) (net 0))
 (segment (start 101.19 52.705) (end 102.743 52.705) (width 0.25) (layer F.Cu) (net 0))
 (segment (start 99.94 52.705) (end 101.19 52.705) (width 0.25) (layer F.Cu) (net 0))
 (segment (start 99.94 53.975) (end 102.743 53.975) (width 0.25) (layer F.Cu) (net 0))
 (segment (start 101.19 55.245) (end 102.743 55.245) (width 0.25) (layer F.Cu) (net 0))
 (segment (start 99.94 55.245) (end 101.19 55.245) (width 0.25) (layer F.Cu) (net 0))
 (segment (start 99.94 56.515) (end 102.743 56.515) (width 0.25) (layer F.Cu) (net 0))
 (segment (start 101.19 57.785) (end 102.743 57.785) (width 0.25) (layer F.Cu) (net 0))
 (segment (start 99.94 57.785) (end 101.19 57.785) (width 0.25) (layer F.Cu) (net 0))
 (segment (start 99.94 59.055) (end 102.743 59.055) (width 0.25) (layer F.Cu) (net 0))
 (segment (start 101.19 60.325) (end 102.743 60.325) (width 0.25) (layer F.Cu) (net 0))
 (segment (start 99.94 60.325) (end 101.19 60.325) (width 0.25) (layer F.Cu) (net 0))
 (segment (start 101.19 61.595) (end 102.743 61.595) (width 0.25) (layer F.Cu) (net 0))
 (segment (start 99.94 61.595) (end 101.19 61.595) (width 0.25) (layer F.Cu) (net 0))
 (segment (start 102.473 62.595) (end 102.743 62.865) (width 0.25) (layer F.Cu) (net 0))
 (segment (start 97.155 62.595) (end 102.473 62.595) (width 0.25) (layer F.Cu) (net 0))
 (segment (start 102.035894 64.135) (end 102.743 64.135) (width 0.25) (layer F.Cu) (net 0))
 (segment (start 96.175 64.135) (end 102.035894 64.135) (width 0.25) (layer F.Cu) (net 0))
 (segment (start 95.885 63.845) (end 96.175 64.135) (width 0.25) (layer F.Cu) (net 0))
 (segment (start 95.885 62.595) (end 95.885 63.845) (width 0.25) (layer F.Cu) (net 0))
 (segment (start 95.123 65.405) (end 102.743 65.405) (width 0.25) (layer F.Cu) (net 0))
 (segment (start 94.615 62.595) (end 94.615 64.897) (width 0.25) (layer F.Cu) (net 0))
 (segment (start 94.615 64.897) (end 95.123 65.405) (width 0.25) (layer F.Cu) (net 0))
 (segment (start 94.488 66.675) (end 102.743 66.675) (width 0.25) (layer F.Cu) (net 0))
 (segment (start 93.345 62.595) (end 93.345 65.532) (width 0.25) (layer F.Cu) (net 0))
 (segment (start 93.345 65.532) (end 94.488 66.675) (width 0.25) (layer F.Cu) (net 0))
 (segment (start 93.472 67.945) (end 102.743 67.945) (width 0.25) (layer F.Cu) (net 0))
 (segment (start 92.075 62.595) (end 92.075 66.548) (width 0.25) (layer F.Cu) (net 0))
 (segment (start 92.075 66.548) (end 93.472 67.945) (width 0.25) (layer F.Cu) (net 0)))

